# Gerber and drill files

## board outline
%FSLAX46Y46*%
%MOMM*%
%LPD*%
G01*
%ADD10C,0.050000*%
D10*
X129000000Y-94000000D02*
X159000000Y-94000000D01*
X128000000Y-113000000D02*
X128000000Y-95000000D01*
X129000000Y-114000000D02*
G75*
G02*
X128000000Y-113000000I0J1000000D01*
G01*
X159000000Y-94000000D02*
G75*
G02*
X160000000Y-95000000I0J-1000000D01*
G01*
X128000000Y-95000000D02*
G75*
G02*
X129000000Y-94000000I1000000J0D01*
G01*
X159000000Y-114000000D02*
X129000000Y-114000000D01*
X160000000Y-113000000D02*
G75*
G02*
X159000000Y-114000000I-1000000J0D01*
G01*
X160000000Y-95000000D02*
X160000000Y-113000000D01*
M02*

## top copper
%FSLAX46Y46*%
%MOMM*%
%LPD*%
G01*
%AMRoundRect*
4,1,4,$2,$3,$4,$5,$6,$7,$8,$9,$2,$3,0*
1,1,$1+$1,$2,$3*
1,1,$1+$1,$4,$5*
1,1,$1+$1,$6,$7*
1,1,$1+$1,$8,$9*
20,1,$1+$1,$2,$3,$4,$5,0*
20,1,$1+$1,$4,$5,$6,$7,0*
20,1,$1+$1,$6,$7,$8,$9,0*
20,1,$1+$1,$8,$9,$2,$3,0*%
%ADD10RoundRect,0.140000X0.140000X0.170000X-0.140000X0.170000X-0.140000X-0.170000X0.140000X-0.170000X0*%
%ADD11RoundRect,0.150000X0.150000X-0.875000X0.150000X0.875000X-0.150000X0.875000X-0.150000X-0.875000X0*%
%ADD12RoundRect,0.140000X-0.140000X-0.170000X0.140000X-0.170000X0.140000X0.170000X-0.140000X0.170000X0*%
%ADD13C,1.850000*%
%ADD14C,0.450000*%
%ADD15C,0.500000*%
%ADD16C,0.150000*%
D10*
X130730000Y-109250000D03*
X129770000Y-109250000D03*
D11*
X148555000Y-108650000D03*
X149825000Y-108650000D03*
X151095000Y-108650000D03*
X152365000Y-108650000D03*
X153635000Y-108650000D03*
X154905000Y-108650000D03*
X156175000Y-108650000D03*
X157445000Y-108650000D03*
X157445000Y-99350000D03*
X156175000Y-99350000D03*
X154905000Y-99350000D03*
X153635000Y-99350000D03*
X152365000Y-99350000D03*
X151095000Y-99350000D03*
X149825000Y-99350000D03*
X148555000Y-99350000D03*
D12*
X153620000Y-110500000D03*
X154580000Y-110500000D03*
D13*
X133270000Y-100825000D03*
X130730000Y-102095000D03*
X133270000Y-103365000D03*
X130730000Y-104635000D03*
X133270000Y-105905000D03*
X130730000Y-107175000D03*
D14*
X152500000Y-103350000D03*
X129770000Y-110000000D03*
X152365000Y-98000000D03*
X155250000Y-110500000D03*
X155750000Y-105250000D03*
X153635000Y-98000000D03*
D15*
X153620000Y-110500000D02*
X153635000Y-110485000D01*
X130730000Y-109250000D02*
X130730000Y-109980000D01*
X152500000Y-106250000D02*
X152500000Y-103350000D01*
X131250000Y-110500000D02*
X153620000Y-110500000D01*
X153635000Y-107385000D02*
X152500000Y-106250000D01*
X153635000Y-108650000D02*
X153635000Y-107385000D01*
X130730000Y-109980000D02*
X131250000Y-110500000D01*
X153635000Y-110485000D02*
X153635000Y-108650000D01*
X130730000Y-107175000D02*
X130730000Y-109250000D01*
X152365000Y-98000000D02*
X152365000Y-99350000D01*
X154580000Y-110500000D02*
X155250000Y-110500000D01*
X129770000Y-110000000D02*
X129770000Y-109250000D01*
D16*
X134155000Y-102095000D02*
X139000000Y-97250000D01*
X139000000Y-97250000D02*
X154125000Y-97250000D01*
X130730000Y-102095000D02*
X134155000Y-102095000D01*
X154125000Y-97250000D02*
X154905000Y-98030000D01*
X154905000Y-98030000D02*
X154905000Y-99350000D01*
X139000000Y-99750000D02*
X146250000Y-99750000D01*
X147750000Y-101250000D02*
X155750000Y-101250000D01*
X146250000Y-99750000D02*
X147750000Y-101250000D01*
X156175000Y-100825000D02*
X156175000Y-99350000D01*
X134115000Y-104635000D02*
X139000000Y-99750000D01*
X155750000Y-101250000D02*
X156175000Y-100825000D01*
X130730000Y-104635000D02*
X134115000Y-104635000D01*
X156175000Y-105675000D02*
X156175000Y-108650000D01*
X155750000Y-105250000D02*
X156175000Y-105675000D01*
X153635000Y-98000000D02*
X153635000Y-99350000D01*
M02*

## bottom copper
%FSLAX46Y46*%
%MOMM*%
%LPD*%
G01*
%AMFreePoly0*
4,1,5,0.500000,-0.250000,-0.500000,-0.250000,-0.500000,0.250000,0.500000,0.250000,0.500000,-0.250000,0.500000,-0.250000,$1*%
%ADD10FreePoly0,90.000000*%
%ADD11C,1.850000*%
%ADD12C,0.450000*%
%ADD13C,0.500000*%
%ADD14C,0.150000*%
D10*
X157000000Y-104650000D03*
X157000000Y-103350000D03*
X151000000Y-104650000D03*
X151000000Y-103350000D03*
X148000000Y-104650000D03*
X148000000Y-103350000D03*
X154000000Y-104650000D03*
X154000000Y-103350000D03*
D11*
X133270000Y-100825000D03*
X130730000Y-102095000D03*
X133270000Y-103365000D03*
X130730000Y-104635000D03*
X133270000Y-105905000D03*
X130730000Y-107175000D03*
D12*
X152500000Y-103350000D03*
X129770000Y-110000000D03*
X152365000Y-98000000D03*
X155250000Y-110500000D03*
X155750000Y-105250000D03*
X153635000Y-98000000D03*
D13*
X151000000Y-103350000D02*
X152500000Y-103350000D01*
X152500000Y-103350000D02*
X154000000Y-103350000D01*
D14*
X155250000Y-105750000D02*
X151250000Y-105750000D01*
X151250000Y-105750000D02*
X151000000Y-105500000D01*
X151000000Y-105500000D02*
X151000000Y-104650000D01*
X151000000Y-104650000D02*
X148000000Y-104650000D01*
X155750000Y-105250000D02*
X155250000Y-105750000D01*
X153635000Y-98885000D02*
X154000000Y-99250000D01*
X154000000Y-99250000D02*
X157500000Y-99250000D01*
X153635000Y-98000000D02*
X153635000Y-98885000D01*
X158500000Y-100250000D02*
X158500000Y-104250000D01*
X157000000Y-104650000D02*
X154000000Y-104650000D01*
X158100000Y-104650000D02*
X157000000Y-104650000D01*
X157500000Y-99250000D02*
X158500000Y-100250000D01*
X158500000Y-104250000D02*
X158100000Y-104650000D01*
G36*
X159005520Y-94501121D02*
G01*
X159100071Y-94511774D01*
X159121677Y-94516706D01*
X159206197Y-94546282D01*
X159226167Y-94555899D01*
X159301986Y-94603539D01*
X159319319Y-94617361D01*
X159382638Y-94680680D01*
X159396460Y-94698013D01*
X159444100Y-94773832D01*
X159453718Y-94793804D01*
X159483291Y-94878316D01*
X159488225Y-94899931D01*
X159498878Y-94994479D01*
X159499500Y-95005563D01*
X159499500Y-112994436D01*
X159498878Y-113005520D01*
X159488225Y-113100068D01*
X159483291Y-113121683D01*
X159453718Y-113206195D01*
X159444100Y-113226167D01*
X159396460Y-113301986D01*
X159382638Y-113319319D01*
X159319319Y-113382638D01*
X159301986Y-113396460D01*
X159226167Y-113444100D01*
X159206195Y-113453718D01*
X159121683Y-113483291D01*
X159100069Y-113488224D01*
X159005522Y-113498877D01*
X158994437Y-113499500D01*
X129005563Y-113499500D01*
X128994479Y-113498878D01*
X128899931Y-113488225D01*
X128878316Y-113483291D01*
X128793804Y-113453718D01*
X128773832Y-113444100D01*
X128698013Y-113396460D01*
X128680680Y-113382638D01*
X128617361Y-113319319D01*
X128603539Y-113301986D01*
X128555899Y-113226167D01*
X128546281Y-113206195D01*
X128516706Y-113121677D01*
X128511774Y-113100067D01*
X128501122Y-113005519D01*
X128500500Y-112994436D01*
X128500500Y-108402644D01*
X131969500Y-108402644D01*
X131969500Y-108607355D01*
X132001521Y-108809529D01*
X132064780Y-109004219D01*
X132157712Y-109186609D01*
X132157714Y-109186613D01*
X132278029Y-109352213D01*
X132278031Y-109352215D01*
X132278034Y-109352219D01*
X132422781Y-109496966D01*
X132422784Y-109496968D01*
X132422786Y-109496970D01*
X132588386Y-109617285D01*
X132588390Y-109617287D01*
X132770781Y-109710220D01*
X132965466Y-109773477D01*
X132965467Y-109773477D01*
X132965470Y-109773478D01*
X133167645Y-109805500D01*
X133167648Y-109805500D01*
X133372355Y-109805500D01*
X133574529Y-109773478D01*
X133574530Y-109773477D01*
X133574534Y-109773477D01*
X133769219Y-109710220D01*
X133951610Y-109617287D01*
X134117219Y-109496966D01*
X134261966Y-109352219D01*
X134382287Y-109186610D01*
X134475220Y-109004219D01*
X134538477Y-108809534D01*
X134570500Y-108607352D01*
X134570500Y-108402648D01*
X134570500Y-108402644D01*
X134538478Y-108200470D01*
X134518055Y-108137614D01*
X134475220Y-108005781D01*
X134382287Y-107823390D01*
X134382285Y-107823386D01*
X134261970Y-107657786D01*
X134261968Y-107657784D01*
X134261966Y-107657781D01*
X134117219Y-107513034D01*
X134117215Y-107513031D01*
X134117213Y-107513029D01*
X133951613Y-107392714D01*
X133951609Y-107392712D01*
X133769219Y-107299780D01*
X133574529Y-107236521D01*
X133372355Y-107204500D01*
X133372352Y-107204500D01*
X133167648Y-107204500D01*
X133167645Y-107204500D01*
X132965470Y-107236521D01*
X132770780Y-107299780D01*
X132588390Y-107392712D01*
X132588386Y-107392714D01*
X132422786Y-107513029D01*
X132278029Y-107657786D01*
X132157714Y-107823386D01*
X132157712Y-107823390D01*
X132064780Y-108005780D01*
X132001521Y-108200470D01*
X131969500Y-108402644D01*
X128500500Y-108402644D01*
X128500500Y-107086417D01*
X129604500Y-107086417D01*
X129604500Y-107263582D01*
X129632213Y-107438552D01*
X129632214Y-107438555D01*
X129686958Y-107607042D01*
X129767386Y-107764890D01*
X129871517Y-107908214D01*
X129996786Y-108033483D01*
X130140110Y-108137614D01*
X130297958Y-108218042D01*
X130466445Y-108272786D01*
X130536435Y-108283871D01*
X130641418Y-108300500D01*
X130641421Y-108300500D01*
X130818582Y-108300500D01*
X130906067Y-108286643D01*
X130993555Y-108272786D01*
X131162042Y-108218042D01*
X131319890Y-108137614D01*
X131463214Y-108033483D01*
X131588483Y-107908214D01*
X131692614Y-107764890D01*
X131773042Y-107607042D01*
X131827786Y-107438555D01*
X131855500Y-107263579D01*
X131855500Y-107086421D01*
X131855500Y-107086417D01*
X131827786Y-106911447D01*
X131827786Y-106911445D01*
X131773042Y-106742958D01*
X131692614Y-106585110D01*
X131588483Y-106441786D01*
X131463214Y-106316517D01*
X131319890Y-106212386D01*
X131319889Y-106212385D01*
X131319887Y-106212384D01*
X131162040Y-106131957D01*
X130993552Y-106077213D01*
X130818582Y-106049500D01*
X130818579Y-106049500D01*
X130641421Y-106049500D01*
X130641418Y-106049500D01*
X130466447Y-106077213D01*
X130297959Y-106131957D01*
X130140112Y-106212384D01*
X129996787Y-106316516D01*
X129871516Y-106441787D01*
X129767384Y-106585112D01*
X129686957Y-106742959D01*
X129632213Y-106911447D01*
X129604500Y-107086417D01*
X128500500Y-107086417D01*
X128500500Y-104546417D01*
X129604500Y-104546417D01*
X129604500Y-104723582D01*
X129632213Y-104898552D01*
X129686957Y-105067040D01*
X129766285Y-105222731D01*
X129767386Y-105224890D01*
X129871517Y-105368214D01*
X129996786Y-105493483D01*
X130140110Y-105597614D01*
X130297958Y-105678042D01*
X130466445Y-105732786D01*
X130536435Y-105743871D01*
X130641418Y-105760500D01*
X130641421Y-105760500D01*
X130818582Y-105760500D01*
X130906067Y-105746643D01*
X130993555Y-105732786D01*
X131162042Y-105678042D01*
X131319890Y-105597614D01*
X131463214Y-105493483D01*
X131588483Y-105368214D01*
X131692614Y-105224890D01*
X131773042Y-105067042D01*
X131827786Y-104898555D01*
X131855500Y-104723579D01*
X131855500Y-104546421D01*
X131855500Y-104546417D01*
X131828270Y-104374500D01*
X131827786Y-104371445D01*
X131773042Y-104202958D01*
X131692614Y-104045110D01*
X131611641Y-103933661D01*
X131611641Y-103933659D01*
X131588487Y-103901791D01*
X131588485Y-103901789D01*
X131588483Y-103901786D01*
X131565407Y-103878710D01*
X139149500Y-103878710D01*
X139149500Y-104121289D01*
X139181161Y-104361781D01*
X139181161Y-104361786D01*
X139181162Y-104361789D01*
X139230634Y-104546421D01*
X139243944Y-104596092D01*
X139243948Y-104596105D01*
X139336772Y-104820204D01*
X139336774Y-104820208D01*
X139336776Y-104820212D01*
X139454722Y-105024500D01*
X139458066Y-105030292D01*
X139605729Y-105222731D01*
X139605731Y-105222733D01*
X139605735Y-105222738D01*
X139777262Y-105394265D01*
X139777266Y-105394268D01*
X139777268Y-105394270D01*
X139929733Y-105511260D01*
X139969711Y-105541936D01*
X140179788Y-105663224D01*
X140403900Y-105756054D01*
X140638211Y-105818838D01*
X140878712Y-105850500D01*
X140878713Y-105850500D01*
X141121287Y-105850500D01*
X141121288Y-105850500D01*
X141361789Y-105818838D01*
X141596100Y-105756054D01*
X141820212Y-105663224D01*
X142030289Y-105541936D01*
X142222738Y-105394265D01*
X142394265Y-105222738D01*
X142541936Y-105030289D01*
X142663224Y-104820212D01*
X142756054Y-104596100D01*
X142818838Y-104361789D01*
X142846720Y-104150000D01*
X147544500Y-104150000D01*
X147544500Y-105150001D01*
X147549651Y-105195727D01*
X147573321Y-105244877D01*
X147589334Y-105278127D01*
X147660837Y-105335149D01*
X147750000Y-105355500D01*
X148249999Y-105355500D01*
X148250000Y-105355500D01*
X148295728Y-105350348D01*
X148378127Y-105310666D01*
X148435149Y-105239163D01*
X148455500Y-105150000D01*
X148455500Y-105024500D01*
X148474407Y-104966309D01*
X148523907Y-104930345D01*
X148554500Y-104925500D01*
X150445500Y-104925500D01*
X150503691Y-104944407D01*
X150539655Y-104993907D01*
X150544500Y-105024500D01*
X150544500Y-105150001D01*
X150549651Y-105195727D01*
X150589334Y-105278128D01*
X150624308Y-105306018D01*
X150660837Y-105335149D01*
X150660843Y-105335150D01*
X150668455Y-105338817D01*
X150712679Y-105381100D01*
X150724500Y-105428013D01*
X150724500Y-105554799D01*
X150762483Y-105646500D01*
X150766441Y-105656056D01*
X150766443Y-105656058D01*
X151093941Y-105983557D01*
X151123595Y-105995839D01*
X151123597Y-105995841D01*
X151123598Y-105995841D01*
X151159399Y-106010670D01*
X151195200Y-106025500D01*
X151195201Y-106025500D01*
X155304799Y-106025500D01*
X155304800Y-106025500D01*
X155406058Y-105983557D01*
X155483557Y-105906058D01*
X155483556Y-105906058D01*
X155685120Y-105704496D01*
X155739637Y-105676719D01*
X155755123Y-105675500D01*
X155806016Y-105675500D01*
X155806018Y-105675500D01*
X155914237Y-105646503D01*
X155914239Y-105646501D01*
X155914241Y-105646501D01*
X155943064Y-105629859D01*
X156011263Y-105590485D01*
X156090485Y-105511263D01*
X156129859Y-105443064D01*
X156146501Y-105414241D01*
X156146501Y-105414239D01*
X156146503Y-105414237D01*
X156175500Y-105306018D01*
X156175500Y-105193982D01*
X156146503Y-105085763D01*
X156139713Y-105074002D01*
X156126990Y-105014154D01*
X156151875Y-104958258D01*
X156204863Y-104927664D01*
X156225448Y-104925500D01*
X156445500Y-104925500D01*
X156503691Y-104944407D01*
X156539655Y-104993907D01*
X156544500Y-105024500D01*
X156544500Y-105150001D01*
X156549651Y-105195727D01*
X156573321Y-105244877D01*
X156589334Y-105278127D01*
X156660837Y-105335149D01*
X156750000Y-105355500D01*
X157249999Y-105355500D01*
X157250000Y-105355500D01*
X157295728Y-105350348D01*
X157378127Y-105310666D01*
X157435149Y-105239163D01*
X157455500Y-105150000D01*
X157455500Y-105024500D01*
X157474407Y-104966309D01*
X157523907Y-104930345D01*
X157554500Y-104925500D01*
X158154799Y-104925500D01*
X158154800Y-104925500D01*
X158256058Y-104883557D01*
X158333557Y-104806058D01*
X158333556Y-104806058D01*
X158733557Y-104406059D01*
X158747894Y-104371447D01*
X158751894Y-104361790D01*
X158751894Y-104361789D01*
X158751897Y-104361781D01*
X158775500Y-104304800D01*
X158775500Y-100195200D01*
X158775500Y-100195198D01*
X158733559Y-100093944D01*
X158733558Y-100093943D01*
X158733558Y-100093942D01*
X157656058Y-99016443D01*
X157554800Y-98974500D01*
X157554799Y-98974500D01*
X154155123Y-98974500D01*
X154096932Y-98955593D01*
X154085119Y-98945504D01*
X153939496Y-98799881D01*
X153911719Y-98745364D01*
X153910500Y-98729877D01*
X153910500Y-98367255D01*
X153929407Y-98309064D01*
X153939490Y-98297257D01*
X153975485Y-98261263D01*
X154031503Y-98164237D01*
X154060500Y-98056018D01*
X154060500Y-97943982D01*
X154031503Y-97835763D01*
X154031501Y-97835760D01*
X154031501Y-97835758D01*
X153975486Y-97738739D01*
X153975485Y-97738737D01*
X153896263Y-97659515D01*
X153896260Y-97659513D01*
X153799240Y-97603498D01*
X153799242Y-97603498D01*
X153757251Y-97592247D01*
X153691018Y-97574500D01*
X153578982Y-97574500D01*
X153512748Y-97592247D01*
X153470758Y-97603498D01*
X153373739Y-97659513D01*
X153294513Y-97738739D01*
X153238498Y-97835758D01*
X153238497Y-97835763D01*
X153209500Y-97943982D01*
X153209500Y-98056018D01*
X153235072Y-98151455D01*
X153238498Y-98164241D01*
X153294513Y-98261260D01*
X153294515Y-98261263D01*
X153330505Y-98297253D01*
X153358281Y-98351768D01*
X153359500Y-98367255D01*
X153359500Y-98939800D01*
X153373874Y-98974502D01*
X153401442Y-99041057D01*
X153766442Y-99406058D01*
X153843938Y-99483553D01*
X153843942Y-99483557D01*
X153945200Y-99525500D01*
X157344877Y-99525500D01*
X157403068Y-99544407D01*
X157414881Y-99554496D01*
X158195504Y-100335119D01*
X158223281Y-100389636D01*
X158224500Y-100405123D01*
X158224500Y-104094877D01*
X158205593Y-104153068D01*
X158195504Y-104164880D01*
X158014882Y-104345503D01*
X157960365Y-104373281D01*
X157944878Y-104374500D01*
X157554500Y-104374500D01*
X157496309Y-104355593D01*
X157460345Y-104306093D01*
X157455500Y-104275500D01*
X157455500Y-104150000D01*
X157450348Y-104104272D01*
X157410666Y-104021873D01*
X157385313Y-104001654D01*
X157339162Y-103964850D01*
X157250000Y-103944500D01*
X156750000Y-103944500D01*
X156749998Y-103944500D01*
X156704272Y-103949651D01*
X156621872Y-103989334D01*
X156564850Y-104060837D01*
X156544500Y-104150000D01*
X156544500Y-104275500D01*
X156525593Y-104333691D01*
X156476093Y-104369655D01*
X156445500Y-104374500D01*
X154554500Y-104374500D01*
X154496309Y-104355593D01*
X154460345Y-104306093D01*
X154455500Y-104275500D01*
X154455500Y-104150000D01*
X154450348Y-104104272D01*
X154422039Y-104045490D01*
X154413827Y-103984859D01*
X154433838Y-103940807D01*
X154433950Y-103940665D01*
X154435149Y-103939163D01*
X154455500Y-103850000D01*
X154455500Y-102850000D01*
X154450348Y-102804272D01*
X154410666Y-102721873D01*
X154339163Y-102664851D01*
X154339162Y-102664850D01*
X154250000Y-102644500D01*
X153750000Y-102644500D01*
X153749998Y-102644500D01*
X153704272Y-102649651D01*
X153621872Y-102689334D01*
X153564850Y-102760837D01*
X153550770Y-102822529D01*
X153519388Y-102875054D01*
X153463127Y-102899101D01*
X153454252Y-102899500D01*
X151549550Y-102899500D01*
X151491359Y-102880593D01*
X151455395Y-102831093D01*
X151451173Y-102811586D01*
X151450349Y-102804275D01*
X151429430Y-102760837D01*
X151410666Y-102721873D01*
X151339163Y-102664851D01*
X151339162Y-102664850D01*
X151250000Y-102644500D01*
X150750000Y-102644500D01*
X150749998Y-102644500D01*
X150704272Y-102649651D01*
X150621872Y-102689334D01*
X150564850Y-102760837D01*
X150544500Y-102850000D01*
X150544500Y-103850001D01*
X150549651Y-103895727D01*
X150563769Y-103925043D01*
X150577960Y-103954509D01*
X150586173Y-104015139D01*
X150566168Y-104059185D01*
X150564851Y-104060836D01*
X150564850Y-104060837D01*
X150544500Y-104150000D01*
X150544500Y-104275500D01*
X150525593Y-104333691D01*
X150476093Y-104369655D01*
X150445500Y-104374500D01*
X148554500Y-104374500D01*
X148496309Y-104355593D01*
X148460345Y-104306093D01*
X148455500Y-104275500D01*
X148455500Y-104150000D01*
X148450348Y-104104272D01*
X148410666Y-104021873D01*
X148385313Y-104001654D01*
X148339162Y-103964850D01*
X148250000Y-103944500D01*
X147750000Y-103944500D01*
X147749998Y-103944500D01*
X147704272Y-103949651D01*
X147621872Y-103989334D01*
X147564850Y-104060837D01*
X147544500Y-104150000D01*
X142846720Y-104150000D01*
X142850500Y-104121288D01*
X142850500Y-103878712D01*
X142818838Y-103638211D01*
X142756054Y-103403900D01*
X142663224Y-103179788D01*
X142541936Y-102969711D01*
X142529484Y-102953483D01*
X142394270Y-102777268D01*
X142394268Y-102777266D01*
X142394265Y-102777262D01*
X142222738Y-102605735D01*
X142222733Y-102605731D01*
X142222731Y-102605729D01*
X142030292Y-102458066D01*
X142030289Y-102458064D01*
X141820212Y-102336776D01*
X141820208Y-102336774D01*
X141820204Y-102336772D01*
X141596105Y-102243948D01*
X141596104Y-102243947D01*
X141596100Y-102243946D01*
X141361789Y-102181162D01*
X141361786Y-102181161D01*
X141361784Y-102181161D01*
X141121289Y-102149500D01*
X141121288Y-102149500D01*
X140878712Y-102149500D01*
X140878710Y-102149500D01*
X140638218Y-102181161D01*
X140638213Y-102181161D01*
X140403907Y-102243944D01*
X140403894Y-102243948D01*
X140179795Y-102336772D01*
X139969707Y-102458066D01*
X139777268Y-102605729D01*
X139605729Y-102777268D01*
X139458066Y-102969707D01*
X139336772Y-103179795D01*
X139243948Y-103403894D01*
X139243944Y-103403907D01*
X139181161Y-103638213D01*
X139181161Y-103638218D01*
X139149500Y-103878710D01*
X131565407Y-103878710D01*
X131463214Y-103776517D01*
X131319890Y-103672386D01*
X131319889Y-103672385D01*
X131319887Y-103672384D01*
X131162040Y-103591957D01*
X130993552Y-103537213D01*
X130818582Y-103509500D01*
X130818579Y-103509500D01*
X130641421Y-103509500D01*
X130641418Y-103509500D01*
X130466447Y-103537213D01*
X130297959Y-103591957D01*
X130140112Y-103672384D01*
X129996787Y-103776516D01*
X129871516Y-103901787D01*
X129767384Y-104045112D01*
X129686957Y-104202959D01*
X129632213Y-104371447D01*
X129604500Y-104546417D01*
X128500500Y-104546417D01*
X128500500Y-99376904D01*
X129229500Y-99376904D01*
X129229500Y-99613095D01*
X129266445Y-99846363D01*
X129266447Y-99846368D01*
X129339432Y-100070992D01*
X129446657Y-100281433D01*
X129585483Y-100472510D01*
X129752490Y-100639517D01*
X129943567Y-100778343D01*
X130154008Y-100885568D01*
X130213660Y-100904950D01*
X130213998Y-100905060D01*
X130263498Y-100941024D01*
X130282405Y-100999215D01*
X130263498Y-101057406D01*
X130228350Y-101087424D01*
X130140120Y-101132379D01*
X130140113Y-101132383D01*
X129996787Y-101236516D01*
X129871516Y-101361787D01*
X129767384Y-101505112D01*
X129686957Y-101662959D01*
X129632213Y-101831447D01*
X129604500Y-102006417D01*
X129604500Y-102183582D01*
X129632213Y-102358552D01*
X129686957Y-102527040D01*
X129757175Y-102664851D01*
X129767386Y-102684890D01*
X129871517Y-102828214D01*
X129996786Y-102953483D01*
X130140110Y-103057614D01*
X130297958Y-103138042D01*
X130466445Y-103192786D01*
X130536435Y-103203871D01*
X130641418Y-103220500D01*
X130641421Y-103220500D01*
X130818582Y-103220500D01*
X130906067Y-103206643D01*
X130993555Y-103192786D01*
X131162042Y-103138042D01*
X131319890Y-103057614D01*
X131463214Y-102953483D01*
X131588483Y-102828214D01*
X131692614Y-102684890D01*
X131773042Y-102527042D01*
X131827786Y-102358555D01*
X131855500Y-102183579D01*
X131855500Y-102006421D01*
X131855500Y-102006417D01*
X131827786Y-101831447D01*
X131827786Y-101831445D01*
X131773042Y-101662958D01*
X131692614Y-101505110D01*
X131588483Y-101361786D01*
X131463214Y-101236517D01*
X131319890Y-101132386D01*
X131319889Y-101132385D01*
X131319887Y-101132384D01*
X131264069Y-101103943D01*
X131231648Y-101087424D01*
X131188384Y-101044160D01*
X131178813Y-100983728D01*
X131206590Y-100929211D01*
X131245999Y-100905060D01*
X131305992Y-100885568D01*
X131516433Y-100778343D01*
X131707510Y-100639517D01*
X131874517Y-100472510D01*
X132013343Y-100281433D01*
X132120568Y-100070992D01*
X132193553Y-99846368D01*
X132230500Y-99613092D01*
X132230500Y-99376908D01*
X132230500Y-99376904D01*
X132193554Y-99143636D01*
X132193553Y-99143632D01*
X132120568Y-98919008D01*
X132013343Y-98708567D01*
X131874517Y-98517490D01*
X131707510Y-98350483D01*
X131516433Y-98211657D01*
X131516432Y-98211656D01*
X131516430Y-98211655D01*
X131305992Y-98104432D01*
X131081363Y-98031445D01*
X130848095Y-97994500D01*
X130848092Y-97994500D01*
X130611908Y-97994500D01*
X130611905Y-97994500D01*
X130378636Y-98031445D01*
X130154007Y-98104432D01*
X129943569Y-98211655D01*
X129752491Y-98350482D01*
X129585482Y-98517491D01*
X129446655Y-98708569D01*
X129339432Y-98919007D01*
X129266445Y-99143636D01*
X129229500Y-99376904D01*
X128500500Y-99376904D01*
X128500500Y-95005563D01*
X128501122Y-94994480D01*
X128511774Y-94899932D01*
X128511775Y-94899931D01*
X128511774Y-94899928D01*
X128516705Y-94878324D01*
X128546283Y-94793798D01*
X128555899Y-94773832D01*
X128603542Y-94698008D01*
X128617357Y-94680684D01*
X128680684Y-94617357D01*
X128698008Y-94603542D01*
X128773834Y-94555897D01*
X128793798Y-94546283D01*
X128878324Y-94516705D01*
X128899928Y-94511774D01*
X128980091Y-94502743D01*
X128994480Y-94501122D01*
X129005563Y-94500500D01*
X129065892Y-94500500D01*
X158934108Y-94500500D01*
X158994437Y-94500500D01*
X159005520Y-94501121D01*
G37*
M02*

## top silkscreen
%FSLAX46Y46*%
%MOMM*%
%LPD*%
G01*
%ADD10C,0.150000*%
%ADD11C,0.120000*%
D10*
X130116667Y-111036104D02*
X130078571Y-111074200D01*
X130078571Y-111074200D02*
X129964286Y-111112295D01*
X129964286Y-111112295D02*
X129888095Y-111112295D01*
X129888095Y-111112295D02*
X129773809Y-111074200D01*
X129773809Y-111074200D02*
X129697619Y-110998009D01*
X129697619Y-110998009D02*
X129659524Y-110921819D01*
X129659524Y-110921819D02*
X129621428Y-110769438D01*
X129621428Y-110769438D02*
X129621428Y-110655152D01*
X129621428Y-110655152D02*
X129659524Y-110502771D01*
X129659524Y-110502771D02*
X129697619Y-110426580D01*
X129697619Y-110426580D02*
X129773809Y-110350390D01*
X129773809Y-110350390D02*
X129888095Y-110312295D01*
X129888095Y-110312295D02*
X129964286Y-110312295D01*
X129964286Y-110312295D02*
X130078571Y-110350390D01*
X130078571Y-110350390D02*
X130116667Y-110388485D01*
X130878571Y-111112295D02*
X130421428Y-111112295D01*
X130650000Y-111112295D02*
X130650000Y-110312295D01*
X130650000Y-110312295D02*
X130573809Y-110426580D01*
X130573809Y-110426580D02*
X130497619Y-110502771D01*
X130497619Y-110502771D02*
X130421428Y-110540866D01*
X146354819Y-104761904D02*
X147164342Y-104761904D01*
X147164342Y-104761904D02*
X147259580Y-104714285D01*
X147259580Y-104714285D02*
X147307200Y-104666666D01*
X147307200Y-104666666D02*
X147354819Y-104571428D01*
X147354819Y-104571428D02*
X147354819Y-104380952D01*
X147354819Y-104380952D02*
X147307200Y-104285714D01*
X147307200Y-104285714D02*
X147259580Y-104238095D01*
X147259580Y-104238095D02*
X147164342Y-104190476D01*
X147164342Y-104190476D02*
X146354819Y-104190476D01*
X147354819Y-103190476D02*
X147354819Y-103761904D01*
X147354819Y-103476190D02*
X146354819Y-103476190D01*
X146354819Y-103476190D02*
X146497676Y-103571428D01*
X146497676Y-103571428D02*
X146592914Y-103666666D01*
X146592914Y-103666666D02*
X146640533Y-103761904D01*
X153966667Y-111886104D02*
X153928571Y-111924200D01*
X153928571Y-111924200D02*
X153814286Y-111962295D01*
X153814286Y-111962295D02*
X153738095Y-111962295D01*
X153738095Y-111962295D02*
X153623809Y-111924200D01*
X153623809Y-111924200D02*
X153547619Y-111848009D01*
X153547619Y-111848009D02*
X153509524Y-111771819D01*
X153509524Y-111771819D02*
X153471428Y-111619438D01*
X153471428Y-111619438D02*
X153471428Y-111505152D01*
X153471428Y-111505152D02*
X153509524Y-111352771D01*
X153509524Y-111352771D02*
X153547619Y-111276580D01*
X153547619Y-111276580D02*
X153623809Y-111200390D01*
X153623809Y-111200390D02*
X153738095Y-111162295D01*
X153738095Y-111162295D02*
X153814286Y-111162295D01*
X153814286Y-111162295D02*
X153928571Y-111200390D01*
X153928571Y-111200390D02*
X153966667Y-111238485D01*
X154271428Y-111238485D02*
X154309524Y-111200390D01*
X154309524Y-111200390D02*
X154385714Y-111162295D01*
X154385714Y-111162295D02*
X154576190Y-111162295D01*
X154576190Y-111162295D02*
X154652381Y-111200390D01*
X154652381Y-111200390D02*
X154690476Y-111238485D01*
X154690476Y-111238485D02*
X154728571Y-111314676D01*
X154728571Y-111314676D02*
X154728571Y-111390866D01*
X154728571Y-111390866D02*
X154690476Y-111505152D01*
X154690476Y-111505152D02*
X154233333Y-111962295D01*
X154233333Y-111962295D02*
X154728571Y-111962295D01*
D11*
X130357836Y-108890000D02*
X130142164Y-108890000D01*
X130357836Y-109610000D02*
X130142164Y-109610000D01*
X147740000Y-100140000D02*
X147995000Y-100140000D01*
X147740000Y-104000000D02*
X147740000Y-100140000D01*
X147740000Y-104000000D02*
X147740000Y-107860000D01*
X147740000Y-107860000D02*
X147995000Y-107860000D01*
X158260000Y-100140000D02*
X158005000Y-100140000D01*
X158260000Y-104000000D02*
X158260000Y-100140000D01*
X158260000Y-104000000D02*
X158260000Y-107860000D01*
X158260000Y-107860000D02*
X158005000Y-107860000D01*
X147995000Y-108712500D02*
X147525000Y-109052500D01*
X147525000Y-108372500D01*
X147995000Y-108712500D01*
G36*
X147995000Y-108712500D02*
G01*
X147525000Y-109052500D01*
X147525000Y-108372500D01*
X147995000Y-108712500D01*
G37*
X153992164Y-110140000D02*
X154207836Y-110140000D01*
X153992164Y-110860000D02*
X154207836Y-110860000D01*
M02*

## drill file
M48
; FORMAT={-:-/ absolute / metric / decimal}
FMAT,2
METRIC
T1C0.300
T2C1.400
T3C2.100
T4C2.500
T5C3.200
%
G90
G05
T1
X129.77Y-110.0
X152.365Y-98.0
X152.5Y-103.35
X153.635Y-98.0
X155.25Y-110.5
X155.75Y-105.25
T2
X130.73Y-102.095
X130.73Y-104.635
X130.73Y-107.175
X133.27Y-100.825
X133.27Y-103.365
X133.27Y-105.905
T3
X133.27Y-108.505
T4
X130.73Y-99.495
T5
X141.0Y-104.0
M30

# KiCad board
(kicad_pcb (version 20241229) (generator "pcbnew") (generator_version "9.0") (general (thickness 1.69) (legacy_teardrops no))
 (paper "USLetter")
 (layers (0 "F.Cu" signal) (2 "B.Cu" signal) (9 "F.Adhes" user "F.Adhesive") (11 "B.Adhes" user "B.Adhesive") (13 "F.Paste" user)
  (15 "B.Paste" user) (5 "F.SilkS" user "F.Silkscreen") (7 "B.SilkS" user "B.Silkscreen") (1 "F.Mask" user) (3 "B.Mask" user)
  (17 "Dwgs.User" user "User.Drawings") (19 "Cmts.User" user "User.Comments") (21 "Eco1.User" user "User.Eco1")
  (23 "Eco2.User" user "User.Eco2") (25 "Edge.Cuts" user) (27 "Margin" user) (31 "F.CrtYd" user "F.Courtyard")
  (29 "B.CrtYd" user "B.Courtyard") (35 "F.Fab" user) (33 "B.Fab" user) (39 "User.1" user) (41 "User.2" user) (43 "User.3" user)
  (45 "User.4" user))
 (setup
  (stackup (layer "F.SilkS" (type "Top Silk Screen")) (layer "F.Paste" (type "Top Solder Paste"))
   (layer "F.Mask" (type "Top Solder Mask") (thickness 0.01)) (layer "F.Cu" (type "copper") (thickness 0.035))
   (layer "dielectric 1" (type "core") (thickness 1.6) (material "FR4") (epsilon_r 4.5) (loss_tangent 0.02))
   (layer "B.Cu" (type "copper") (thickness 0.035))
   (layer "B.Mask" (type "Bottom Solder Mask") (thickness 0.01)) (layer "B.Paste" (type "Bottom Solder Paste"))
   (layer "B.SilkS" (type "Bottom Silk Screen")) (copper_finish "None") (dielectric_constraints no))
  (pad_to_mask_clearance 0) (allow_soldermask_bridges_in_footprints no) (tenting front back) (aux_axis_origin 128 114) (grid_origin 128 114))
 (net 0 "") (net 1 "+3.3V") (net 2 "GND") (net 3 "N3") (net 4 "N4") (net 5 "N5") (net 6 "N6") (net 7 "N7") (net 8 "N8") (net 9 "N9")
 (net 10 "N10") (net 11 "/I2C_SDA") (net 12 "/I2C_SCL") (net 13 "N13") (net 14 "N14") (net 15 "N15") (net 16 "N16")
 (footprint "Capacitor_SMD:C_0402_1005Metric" (layer "F.Cu") (at 130.25 109.25 180)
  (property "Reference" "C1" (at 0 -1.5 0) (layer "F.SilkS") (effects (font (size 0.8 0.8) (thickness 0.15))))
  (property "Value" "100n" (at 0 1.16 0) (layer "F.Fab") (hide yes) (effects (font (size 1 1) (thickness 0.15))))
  (fp_line (start -0.107836 0.36) (end 0.107836 0.36) (stroke (width 0.12) (type solid)) (layer "F.SilkS"))
  (fp_line (start -0.107836 -0.36) (end 0.107836 -0.36) (stroke (width 0.12) (type solid)) (layer "F.SilkS"))
  (pad "1" smd roundrect (at -0.48 0 180) (size 0.56 0.62) (layers "F.Cu" "F.Mask" "F.Paste") (roundrect_rratio 0.25) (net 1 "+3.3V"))
  (pad "2" smd roundrect (at 0.48 0 180) (size 0.56 0.62) (layers "F.Cu" "F.Mask" "F.Paste") (roundrect_rratio 0.25) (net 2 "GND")))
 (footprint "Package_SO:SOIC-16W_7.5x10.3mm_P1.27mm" (layer "F.Cu") (at 153 104 90)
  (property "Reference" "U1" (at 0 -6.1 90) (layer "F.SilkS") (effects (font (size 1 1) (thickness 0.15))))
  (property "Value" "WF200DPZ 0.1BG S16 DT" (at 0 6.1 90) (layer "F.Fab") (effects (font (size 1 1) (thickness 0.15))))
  (fp_line (start 3.86 -5.26) (end 3.86 -5.005) (stroke (width 0.12) (type solid)) (layer "F.SilkS"))
  (fp_line (start 0 -5.26) (end 3.86 -5.26) (stroke (width 0.12) (type solid)) (layer "F.SilkS"))
  (fp_line (start 0 -5.26) (end -3.86 -5.26) (stroke (width 0.12) (type solid)) (layer "F.SilkS"))
  (fp_line (start -3.86 -5.26) (end -3.86 -5.005) (stroke (width 0.12) (type solid)) (layer "F.SilkS"))
  (fp_line (start 3.86 5.26) (end 3.86 5.005) (stroke (width 0.12) (type solid)) (layer "F.SilkS"))
  (fp_line (start 0 5.26) (end 3.86 5.26) (stroke (width 0.12) (type solid)) (layer "F.SilkS"))
  (fp_line (start 0 5.26) (end -3.86 5.26) (stroke (width 0.12) (type solid)) (layer "F.SilkS"))
  (fp_line (start -3.86 5.26) (end -3.86 5.005) (stroke (width 0.12) (type solid)) (layer "F.SilkS"))
  (fp_poly
   (pts (xy -4.7125 -5.005) (xy -5.0525 -5.475) (xy -4.3725 -5.475)) (stroke (width 0.12) (type solid)) (fill yes) (layer "F.SilkS"))
  (pad "1" smd roundrect (at -4.65 -4.445 90) (size 2.05 0.6) (layers "F.Cu" "F.Mask" "F.Paste") (roundrect_rratio 0.25) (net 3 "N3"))
  (pad "2" smd roundrect (at -4.65 -3.175 90) (size 2.05 0.6) (layers "F.Cu" "F.Mask" "F.Paste") (roundrect_rratio 0.25) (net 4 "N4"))
  (pad "3" smd roundrect (at -4.65 -1.905 90) (size 2.05 0.6) (layers "F.Cu" "F.Mask" "F.Paste") (roundrect_rratio 0.25) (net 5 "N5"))
  (pad "4" smd roundrect (at -4.65 -0.635 90) (size 2.05 0.6) (layers "F.Cu" "F.Mask" "F.Paste") (roundrect_rratio 0.25) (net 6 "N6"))
  (pad "5" smd roundrect (at -4.65 0.635 90) (size 2.05 0.6) (layers "F.Cu" "F.Mask" "F.Paste") (roundrect_rratio 0.25) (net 1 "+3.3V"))
  (pad "6" smd roundrect (at -4.65 1.905 90) (size 2.05 0.6) (layers "F.Cu" "F.Mask" "F.Paste") (roundrect_rratio 0.25) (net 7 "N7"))
  (pad "7" smd roundrect (at -4.65 3.175 90) (size 2.05 0.6) (layers "F.Cu" "F.Mask" "F.Paste") (roundrect_rratio 0.25) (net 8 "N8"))
  (pad "8" smd roundrect (at -4.65 4.445 90) (size 2.05 0.6) (layers "F.Cu" "F.Mask" "F.Paste") (roundrect_rratio 0.25) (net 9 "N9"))
  (pad "9" smd roundrect (at 4.65 4.445 90) (size 2.05 0.6) (layers "F.Cu" "F.Mask" "F.Paste") (roundrect_rratio 0.25) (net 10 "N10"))
  (pad "10" smd roundrect (at 4.65 3.175 90) (size 2.05 0.6) (layers "F.Cu" "F.Mask" "F.Paste") (roundrect_rratio 0.25) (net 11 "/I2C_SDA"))
  (pad "11" smd roundrect (at 4.65 1.905 90) (size 2.05 0.6) (layers "F.Cu" "F.Mask" "F.Paste") (roundrect_rratio 0.25) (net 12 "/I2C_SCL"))
  (pad "12" smd roundrect (at 4.65 0.635 90) (size 2.05 0.6) (layers "F.Cu" "F.Mask" "F.Paste") (roundrect_rratio 0.25) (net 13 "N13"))
  (pad "13" smd roundrect (at 4.65 -0.635 90) (size 2.05 0.6) (layers "F.Cu" "F.Mask" "F.Paste") (roundrect_rratio 0.25) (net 2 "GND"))
  (pad "14" smd roundrect (at 4.65 -1.905 90) (size 2.05 0.6) (layers "F.Cu" "F.Mask" "F.Paste") (roundrect_rratio 0.25) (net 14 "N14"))
  (pad "15" smd roundrect (at 4.65 -3.175 90) (size 2.05 0.6) (layers "F.Cu" "F.Mask" "F.Paste") (roundrect_rratio 0.25) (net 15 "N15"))
  (pad "16" smd roundrect (at 4.65 -4.445 90) (size 2.05 0.6) (layers "F.Cu" "F.Mask" "F.Paste") (roundrect_rratio 0.25) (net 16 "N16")))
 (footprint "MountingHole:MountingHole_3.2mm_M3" (layer "F.Cu") (at 141 104)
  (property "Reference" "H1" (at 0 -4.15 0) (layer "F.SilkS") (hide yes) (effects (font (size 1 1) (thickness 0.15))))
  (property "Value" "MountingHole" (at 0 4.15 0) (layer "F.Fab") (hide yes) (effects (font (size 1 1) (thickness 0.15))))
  (pad "" np_thru_hole circle (at 0 0) (size 3.2 3.2) (drill 3.2) (layers "*.Cu" "*.Mask")))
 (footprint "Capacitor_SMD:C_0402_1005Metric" (layer "F.Cu") (at 154.1 110.5)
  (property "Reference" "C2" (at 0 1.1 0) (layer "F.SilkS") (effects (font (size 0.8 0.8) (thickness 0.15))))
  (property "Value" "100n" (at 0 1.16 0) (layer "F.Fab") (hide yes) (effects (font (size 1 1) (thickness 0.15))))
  (fp_line (start -0.107836 -0.36) (end 0.107836 -0.36) (stroke (width 0.12) (type solid)) (layer "F.SilkS"))
  (fp_line (start -0.107836 0.36) (end 0.107836 0.36) (stroke (width 0.12) (type solid)) (layer "F.SilkS"))
  (pad "1" smd roundrect (at -0.48 0) (size 0.56 0.62) (layers "F.Cu" "F.Mask" "F.Paste") (roundrect_rratio 0.25) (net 1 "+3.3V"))
  (pad "2" smd roundrect (at 0.48 0) (size 0.56 0.62) (layers "F.Cu" "F.Mask" "F.Paste") (roundrect_rratio 0.25) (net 2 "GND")))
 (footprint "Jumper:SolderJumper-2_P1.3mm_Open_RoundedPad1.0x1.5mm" (layer "B.Cu") (at 157 104 90)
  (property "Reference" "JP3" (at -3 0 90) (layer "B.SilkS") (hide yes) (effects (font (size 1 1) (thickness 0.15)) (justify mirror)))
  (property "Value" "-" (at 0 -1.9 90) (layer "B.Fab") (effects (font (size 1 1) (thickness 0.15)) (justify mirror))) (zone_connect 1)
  (pad "1" smd custom (at -0.65 0 90) (size 1 0.5) (layers "B.Cu" "B.Mask") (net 13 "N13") (zone_connect 2) (thermal_bridge_angle 45)
   (options (clearance outline) (anchor rect)) (primitives))
  (pad "2" smd custom (at 0.65 0 90) (size 1 0.5) (layers "B.Cu" "B.Mask") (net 2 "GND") (zone_connect 2) (thermal_bridge_angle 45)
   (options (clearance outline) (anchor rect)) (primitives)))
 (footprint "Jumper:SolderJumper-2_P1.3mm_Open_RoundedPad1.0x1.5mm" (layer "B.Cu") (at 151 104 90)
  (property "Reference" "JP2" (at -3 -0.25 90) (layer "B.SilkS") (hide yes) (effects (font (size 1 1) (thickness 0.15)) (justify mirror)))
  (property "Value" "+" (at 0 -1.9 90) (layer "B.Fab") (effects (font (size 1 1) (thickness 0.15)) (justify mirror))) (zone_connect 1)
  (pad "1" smd custom (at -0.65 0 90) (size 1 0.5) (layers "B.Cu" "B.Mask") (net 8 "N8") (zone_connect 2) (thermal_bridge_angle 45)
   (options (clearance outline) (anchor rect)) (primitives))
  (pad "2" smd custom (at 0.65 0 90) (size 1 0.5) (layers "B.Cu" "B.Mask") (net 1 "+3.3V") (zone_connect 2) (thermal_bridge_angle 45)
   (options (clearance outline) (anchor rect)) (primitives)))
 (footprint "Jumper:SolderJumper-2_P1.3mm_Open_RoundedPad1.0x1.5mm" (layer "B.Cu") (at 148 104 90)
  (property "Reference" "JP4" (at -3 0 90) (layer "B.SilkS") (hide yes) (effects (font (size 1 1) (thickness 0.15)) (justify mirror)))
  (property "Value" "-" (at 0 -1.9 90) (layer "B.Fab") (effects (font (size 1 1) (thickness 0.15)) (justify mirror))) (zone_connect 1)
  (pad "1" smd custom (at -0.65 0 90) (size 1 0.5) (layers "B.Cu" "B.Mask") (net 8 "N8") (zone_connect 2) (thermal_bridge_angle 45)
   (options (clearance outline) (anchor rect)) (primitives))
  (pad "2" smd custom (at 0.65 0 90) (size 1 0.5) (layers "B.Cu" "B.Mask") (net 2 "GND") (zone_connect 2) (thermal_bridge_angle 45)
   (options (clearance outline) (anchor rect)) (primitives)))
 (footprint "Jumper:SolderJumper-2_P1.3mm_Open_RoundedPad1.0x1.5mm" (layer "B.Cu") (at 154 104 90)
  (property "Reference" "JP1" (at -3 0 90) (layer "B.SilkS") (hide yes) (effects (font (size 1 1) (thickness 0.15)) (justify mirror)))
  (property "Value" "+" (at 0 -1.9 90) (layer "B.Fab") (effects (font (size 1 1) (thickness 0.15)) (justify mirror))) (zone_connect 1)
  (pad "1" smd custom (at -0.65 0 90) (size 1 0.5) (layers "B.Cu" "B.Mask") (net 13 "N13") (zone_connect 2) (thermal_bridge_angle 45)
   (options (clearance outline) (anchor rect)) (primitives))
  (pad "2" smd custom (at 0.65 0 90) (size 1 0.5) (layers "B.Cu" "B.Mask") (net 1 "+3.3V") (zone_connect 2) (thermal_bridge_angle 45)
   (options (clearance outline) (anchor rect)) (primitives)))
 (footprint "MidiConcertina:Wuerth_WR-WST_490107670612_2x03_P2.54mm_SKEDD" (layer "B.Cu") (at 132 104 180)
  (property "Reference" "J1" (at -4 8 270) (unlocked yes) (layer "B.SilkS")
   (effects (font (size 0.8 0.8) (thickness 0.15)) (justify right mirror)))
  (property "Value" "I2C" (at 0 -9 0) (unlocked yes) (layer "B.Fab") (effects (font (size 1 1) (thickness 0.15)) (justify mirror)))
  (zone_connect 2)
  (pad "" np_thru_hole circle (at -1.27 -4.505 180) (size 2.1 2.1) (drill 2.1) (layers "*.Cu" "*.Mask"))
  (pad "" np_thru_hole circle (at 1.27 4.505 180) (size 2.5 2.5) (drill 2.5) (layers "*.Cu" "*.Mask"))
  (pad "1" thru_hole circle (at -1.27 3.175 180) (size 1.85 1.85) (drill 1.4) (layers "*.Cu" "*.Mask") (remove_unused_layers no)
   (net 2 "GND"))
  (pad "2" thru_hole circle (at 1.27 1.905 180) (size 1.85 1.85) (drill 1.4) (layers "*.Cu" "*.Mask") (remove_unused_layers no)
   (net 12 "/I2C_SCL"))
  (pad "3" thru_hole circle (at -1.27 0.635 180) (size 1.85 1.85) (drill 1.4) (layers "*.Cu" "*.Mask") (remove_unused_layers no)
   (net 2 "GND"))
  (pad "4" thru_hole circle (at 1.27 -0.635 180) (size 1.85 1.85) (drill 1.4) (layers "*.Cu" "*.Mask") (remove_unused_layers no)
   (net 11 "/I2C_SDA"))
  (pad "5" thru_hole circle (at -1.27 -1.905 180) (size 1.85 1.85) (drill 1.4) (layers "*.Cu" "*.Mask") (remove_unused_layers no)
   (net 2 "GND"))
  (pad "6" thru_hole circle (at 1.27 -3.175 180) (size 1.85 1.85) (drill 1.4) (layers "*.Cu" "*.Mask") (remove_unused_layers no)
   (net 1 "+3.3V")))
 (gr_line (start 129 94) (end 159 94) (stroke (width 0.05) (type default)) (layer "Edge.Cuts"))
 (gr_line (start 128 113) (end 128 95) (stroke (width 0.05) (type default)) (layer "Edge.Cuts"))
 (gr_arc (start 129 114) (mid 128.292893 113.707107) (end 128 113) (stroke (width 0.05) (type default)) (layer "Edge.Cuts"))
 (gr_arc (start 159 94) (mid 159.707107 94.292893) (end 160 95) (stroke (width 0.05) (type default)) (layer "Edge.Cuts"))
 (gr_arc (start 128 95) (mid 128.292893 94.292893) (end 129 94) (stroke (width 0.05) (type default)) (layer "Edge.Cuts"))
 (gr_line (start 159 114) (end 129 114) (stroke (width 0.05) (type default)) (layer "Edge.Cuts"))
 (gr_arc (start 160 113) (mid 159.707107 113.707107) (end 159 114) (stroke (width 0.05) (type default)) (layer "Edge.Cuts"))
 (gr_line (start 160 95) (end 160 113) (stroke (width 0.05) (type default)) (layer "Edge.Cuts"))
 (segment (start 153.62 110.5) (end 153.635 110.485) (width 0.5) (layer "F.Cu") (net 1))
 (segment (start 130.73 109.25) (end 130.73 109.98) (width 0.5) (layer "F.Cu") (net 1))
 (segment (start 152.5 106.25) (end 152.5 103.35) (width 0.5) (layer "F.Cu") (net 1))
 (segment (start 131.25 110.5) (end 153.62 110.5) (width 0.5) (layer "F.Cu") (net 1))
 (segment (start 153.635 107.385) (end 152.5 106.25) (width 0.5) (layer "F.Cu") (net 1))
 (segment (start 153.635 108.65) (end 153.635 107.385) (width 0.5) (layer "F.Cu") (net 1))
 (segment (start 130.73 109.98) (end 131.25 110.5) (width 0.5) (layer "F.Cu") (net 1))
 (segment (start 153.635 110.485) (end 153.635 108.65) (width 0.5) (layer "F.Cu") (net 1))
 (segment (start 130.73 107.175) (end 130.73 109.25) (width 0.5) (layer "F.Cu") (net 1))
 (via (at 152.5 103.35) (size 0.45) (drill 0.3) (layers "F.Cu" "B.Cu") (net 1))
 (segment (start 151 103.35) (end 152.5 103.35) (width 0.5) (layer "B.Cu") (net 1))
 (segment (start 152.5 103.35) (end 154 103.35) (width 0.5) (layer "B.Cu") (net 1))
 (segment (start 152.365 98) (end 152.365 99.35) (width 0.5) (layer "F.Cu") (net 2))
 (segment (start 154.58 110.5) (end 155.25 110.5) (width 0.5) (layer "F.Cu") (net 2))
 (segment (start 129.77 110) (end 129.77 109.25) (width 0.5) (layer "F.Cu") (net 2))
 (via (at 129.77 110) (size 0.45) (drill 0.3) (layers "F.Cu" "B.Cu") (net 2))
 (via (at 152.365 98) (size 0.45) (drill 0.3) (layers "F.Cu" "B.Cu") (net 2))
 (via (at 155.25 110.5) (size 0.45) (drill 0.3) (layers "F.Cu" "B.Cu") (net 2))
 (segment (start 134.155 102.095) (end 139 97.25) (width 0.15) (layer "F.Cu") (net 12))
 (segment (start 139 97.25) (end 154.125 97.25) (width 0.15) (layer "F.Cu") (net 12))
 (segment (start 130.73 102.095) (end 134.155 102.095) (width 0.15) (layer "F.Cu") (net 12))
 (segment (start 154.125 97.25) (end 154.905 98.03) (width 0.15) (layer "F.Cu") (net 12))
 (segment (start 154.905 98.03) (end 154.905 99.35) (width 0.15) (layer "F.Cu") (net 12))
 (segment (start 139 99.75) (end 146.25 99.75) (width 0.15) (layer "F.Cu") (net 11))
 (segment (start 147.75 101.25) (end 155.75 101.25) (width 0.15) (layer "F.Cu") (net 11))
 (segment (start 146.25 99.75) (end 147.75 101.25) (width 0.15) (layer "F.Cu") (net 11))
 (segment (start 156.175 100.825) (end 156.175 99.35) (width 0.15) (layer "F.Cu") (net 11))
 (segment (start 134.115 104.635) (end 139 99.75) (width 0.15) (layer "F.Cu") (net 11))
 (segment (start 155.75 101.25) (end 156.175 100.825) (width 0.15) (layer "F.Cu") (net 11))
 (segment (start 130.73 104.635) (end 134.115 104.635) (width 0.15) (layer "F.Cu") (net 11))
 (segment (start 156.175 105.675) (end 156.175 108.65) (width 0.15) (layer "F.Cu") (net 8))
 (segment (start 155.75 105.25) (end 156.175 105.675) (width 0.15) (layer "F.Cu") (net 8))
 (via (at 155.75 105.25) (size 0.45) (drill 0.3) (layers "F.Cu" "B.Cu") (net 8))
 (segment (start 155.25 105.75) (end 151.25 105.75) (width 0.15) (layer "B.Cu") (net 8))
 (segment (start 151.25 105.75) (end 151 105.5) (width 0.15) (layer "B.Cu") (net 8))
 (segment (start 151 105.5) (end 151 104.65) (width 0.15) (layer "B.Cu") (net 8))
 (segment (start 151 104.65) (end 148 104.65) (width 0.15) (layer "B.Cu") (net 8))
 (segment (start 155.75 105.25) (end 155.25 105.75) (width 0.15) (layer "B.Cu") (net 8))
 (segment (start 153.635 98) (end 153.635 99.35) (width 0.15) (layer "F.Cu") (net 13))
 (via (at 153.635 98) (size 0.45) (drill 0.3) (layers "F.Cu" "B.Cu") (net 13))
 (segment (start 153.635 98.885) (end 154 99.25) (width 0.15) (layer "B.Cu") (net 13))
 (segment (start 154 99.25) (end 157.5 99.25) (width 0.15) (layer "B.Cu") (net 13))
 (segment (start 153.635 98) (end 153.635 98.885) (width 0.15) (layer "B.Cu") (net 13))
 (segment (start 158.5 100.25) (end 158.5 104.25) (width 0.15) (layer "B.Cu") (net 13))
 (segment (start 157 104.65) (end 154 104.65) (width 0.15) (layer "B.Cu") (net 13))
 (segment (start 158.1 104.65) (end 157 104.65) (width 0.15) (layer "B.Cu") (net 13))
 (segment (start 157.5 99.25) (end 158.5 100.25) (width 0.15) (layer "B.Cu") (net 13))
 (segment (start 158.5 104.25) (end 158.1 104.65) (width 0.15) (layer "B.Cu") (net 13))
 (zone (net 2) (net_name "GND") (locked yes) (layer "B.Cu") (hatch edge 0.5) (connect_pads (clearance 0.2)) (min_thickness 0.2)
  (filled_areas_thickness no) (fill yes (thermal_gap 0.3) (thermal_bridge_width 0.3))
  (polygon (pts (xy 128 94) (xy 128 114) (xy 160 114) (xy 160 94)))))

